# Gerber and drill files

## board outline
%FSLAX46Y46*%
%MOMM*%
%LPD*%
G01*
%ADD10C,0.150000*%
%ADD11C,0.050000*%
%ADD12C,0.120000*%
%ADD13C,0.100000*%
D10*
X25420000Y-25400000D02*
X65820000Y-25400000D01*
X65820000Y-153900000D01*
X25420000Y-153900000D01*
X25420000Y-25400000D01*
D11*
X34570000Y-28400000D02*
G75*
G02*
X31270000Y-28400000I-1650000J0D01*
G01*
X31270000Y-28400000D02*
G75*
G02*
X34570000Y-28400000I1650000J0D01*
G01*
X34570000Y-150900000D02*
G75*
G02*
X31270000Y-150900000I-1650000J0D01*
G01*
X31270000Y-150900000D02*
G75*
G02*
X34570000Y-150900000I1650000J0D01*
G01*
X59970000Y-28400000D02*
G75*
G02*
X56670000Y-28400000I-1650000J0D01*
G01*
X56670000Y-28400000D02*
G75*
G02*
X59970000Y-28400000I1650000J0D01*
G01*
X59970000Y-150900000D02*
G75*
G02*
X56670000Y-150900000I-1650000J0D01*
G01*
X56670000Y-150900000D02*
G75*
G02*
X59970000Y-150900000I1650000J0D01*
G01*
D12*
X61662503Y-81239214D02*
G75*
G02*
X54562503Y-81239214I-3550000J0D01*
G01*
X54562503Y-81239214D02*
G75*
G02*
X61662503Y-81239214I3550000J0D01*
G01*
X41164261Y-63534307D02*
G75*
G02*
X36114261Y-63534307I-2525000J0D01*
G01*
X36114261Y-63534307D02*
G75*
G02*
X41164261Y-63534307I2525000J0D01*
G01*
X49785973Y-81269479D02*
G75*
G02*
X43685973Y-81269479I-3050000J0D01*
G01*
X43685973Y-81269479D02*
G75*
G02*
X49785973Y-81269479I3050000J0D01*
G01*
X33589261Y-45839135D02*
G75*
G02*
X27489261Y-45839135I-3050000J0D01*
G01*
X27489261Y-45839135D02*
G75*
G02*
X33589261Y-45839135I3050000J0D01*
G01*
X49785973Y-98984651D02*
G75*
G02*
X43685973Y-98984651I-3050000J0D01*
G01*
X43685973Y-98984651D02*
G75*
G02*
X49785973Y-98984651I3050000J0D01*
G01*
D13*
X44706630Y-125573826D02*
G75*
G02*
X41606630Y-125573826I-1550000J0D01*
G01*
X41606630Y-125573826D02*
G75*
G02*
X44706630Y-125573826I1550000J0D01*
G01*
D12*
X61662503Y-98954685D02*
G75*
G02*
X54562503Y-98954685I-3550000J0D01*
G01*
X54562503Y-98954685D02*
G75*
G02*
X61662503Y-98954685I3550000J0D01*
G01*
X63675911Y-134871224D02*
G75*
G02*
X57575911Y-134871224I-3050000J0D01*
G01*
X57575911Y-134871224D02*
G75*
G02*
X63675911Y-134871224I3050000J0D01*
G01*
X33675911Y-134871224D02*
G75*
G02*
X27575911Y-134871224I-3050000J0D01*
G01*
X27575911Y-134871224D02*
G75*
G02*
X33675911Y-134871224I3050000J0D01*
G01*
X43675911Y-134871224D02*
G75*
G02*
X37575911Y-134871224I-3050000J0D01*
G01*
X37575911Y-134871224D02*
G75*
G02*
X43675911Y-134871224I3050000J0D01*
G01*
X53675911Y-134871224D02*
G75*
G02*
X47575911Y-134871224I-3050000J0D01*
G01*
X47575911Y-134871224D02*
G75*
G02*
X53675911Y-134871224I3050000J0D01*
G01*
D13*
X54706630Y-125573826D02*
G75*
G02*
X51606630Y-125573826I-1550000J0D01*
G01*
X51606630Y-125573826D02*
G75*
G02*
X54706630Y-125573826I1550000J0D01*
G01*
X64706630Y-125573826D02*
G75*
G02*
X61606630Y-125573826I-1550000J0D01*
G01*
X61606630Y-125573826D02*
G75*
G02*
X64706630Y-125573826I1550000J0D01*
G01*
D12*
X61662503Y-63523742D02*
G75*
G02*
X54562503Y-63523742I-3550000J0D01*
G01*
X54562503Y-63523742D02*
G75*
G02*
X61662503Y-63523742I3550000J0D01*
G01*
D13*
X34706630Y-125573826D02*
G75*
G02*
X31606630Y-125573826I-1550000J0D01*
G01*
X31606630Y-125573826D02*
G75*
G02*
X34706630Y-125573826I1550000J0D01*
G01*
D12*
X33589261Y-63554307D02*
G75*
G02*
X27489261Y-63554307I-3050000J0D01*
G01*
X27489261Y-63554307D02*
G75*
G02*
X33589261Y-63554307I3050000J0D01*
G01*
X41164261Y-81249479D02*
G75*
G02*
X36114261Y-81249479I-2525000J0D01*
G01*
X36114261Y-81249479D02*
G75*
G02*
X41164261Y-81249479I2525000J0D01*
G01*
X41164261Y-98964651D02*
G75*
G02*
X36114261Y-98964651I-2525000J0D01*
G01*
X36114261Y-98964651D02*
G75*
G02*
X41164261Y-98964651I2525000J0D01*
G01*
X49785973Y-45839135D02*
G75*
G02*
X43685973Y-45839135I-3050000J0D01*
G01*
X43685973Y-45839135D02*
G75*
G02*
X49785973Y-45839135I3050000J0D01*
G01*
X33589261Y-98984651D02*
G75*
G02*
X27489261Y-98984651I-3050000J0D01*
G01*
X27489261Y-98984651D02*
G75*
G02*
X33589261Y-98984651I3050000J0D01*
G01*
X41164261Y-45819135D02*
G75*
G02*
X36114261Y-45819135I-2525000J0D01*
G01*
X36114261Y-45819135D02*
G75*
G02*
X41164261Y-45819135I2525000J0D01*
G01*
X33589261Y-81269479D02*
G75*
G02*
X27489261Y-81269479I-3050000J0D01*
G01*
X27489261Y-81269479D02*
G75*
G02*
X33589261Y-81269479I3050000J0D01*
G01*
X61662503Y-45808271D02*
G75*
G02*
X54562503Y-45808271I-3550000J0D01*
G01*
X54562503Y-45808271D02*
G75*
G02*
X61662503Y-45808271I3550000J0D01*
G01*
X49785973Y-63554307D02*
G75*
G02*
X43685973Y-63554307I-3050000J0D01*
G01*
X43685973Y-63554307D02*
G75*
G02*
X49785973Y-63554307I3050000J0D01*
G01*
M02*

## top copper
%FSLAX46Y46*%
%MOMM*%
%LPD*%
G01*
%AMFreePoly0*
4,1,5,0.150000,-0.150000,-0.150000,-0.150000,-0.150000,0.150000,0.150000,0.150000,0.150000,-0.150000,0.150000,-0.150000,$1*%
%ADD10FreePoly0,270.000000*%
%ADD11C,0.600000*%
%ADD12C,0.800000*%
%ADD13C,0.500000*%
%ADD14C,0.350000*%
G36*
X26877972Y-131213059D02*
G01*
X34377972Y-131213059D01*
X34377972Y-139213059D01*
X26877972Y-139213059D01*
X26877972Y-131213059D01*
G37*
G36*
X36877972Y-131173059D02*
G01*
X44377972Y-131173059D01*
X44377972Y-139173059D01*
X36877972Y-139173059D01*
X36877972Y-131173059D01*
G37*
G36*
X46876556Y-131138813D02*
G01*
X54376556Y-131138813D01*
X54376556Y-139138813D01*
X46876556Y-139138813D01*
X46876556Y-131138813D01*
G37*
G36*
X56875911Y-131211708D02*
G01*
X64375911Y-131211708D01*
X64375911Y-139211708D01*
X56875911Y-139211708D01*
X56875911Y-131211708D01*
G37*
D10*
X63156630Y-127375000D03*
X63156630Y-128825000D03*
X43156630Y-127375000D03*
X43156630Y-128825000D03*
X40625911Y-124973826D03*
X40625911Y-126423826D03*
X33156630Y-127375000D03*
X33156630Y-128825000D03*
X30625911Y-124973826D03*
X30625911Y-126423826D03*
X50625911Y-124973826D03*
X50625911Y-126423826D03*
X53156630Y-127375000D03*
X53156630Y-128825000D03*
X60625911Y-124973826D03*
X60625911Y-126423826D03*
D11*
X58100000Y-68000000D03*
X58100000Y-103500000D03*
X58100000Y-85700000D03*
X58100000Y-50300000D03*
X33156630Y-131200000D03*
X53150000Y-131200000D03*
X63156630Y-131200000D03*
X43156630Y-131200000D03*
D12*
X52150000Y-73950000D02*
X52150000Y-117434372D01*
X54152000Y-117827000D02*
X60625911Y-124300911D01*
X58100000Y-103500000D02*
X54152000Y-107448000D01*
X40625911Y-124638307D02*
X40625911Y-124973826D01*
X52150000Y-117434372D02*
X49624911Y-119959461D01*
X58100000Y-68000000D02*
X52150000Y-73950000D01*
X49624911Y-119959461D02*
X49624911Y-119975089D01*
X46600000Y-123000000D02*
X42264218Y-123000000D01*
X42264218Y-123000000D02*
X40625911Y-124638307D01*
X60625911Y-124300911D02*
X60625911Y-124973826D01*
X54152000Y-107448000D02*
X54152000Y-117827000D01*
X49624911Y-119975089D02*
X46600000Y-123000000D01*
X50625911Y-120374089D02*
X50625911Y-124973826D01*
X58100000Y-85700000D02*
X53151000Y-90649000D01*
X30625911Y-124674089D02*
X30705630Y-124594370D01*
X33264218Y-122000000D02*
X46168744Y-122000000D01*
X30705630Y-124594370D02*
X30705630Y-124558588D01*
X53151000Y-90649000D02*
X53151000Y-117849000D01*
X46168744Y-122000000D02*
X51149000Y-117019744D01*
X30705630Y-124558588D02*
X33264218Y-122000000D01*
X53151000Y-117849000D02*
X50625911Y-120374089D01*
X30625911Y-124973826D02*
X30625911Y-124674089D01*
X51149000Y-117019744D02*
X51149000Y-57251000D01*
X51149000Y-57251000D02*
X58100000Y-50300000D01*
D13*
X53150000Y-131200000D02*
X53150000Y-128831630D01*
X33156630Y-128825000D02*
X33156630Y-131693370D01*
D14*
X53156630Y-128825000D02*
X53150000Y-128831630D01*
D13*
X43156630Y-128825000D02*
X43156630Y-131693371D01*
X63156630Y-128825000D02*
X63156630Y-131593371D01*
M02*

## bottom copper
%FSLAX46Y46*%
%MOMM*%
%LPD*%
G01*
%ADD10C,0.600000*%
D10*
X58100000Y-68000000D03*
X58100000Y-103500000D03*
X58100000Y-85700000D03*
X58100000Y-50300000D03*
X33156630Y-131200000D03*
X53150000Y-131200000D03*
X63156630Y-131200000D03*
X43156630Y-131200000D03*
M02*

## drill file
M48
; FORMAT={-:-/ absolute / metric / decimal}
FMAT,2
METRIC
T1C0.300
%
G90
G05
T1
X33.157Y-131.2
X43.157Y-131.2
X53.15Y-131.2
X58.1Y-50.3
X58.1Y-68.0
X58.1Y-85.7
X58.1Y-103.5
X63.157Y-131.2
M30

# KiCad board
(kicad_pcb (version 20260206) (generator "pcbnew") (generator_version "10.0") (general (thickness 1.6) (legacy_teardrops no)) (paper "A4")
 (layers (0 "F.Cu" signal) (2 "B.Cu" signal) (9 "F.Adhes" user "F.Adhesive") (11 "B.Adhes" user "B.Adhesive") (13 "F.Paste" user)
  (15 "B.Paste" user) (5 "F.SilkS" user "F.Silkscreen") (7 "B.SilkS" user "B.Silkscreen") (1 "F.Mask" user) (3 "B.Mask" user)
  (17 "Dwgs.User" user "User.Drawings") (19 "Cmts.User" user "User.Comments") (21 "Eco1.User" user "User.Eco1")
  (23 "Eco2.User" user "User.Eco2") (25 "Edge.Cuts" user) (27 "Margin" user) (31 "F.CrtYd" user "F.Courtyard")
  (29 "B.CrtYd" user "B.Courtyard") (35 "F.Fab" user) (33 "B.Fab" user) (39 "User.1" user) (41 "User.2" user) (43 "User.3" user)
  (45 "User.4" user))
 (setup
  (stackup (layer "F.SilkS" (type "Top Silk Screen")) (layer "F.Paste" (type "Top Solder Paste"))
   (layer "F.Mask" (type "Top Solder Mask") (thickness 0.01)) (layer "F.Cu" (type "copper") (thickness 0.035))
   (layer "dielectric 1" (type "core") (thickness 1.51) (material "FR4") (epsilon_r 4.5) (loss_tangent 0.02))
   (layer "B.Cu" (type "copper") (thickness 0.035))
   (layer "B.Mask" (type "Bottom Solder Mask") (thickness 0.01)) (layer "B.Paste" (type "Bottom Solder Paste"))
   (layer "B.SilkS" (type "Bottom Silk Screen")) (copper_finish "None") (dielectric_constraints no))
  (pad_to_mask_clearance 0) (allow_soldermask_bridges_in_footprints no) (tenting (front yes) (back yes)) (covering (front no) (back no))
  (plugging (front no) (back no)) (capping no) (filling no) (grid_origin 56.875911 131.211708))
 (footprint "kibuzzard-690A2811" (layer "F.Cu") (at 27.621439 39.2)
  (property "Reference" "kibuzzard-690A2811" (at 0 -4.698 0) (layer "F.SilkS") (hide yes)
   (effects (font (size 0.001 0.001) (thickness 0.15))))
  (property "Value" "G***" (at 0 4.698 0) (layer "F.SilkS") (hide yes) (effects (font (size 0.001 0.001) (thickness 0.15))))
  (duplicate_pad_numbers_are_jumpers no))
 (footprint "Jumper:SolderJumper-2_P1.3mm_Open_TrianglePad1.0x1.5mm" (layer "F.Cu") (at 63.15663 128.1 -90)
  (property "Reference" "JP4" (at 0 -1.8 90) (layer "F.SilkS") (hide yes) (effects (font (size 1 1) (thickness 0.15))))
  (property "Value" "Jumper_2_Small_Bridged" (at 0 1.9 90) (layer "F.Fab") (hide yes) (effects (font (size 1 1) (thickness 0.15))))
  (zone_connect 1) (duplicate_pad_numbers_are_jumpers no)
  (pad "1" smd custom (at -0.725 0 270) (size 0.3 0.3) (layers "F.Cu" "F.Mask") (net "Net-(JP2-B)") (zone_connect 2)
   (thermal_bridge_angle 45) (options (clearance outline) (anchor rect)) (primitives))
  (pad "2" smd custom (at 0.725 0 270) (size 0.3 0.3) (layers "F.Cu" "F.Mask") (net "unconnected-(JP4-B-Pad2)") (zone_connect 2)
   (thermal_bridge_angle 45) (options (clearance outline) (anchor rect)) (primitives)))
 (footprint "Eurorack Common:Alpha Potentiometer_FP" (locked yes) (layer "F.Cu") (at 55.612503 88.849214)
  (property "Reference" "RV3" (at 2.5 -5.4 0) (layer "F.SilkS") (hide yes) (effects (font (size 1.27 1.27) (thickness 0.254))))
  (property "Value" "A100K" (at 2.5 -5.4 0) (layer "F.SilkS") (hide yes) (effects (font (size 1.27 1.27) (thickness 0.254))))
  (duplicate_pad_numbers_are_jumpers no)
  (fp_circle (center 2.5 -7.61) (end 6.05 -7.61) (stroke (width 0.12) (type solid)) (fill no) (layer "Edge.Cuts")))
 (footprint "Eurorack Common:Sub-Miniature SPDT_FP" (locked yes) (layer "F.Cu") (at 38.639261 63.534307 90)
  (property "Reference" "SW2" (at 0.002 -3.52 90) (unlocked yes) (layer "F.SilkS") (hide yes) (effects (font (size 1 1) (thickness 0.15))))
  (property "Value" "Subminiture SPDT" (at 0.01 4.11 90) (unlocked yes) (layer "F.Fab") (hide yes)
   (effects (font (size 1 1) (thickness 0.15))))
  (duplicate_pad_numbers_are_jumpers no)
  (fp_circle (center 0 0) (end 2.525 0) (stroke (width 0.12) (type solid)) (fill no) (layer "Edge.Cuts")))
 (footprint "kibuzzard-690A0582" (layer "F.Cu") (at 41.52 141.85)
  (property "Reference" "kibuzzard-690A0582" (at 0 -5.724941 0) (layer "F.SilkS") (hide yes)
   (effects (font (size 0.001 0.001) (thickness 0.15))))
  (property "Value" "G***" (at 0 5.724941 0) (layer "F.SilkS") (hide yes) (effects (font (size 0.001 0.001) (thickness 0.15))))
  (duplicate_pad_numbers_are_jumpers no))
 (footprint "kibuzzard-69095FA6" (layer "F.Cu") (at 30.670922 113.458966)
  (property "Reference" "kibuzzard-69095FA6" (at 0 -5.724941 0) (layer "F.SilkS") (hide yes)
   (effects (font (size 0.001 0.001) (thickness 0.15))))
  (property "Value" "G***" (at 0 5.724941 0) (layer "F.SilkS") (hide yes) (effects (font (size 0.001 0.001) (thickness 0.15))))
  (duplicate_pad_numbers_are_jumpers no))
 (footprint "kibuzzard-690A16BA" (layer "F.Cu") (at 46.3 113.458966)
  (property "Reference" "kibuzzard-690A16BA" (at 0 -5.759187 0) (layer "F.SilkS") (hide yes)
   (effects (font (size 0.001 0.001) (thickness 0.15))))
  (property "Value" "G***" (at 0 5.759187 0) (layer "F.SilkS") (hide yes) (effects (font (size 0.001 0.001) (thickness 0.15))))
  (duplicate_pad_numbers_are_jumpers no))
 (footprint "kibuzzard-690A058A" (layer "F.Cu") (at 51.53 141.85)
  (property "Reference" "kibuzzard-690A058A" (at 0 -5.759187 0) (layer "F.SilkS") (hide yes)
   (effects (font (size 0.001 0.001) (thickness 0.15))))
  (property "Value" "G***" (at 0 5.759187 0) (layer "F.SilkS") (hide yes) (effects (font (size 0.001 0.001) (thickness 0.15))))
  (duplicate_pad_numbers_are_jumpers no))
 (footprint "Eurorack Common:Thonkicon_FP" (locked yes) (layer "F.Cu") (at 46.735973 74.789479)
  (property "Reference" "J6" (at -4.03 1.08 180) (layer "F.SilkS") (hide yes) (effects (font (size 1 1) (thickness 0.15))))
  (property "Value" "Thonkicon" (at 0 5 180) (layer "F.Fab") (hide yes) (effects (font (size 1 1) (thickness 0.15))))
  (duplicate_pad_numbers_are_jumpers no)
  (fp_circle (center 0 6.48) (end 3.05 6.48) (stroke (width 0.12) (type solid)) (fill no) (layer "Edge.Cuts")))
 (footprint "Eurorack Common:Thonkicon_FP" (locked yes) (layer "F.Cu") (at 30.539261 39.359135)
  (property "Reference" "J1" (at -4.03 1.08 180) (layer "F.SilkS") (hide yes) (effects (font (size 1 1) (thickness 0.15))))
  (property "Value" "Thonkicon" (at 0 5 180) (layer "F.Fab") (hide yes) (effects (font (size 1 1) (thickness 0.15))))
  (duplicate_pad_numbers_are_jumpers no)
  (fp_circle (center 0 6.48) (end 3.05 6.48) (stroke (width 0.12) (type solid)) (fill no) (layer "Edge.Cuts")))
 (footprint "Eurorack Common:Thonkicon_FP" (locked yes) (layer "F.Cu") (at 46.735973 92.504651)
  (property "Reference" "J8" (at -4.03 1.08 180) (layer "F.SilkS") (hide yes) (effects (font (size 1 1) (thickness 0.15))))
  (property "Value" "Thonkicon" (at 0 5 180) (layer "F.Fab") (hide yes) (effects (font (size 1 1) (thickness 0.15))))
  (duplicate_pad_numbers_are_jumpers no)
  (fp_circle (center 0 6.48) (end 3.05 6.48) (stroke (width 0.12) (type solid)) (fill no) (layer "Edge.Cuts")))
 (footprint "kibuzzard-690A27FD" (layer "F.Cu") (at 27.429315 56.9)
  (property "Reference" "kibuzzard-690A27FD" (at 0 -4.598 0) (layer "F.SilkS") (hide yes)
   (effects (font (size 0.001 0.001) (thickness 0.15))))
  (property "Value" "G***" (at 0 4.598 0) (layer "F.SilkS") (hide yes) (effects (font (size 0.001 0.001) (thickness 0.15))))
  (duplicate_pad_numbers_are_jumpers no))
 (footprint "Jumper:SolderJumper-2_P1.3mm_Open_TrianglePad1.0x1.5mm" (layer "F.Cu") (at 43.15663 128.1 -90)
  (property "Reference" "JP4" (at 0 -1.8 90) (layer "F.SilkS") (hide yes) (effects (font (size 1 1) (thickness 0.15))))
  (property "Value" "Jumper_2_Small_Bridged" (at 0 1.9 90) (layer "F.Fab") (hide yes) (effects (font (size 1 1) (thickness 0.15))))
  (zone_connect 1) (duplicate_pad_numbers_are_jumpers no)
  (pad "1" smd custom (at -0.725 0 270) (size 0.3 0.3) (layers "F.Cu" "F.Mask") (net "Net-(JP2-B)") (zone_connect 2)
   (thermal_bridge_angle 45) (options (clearance outline) (anchor rect)) (primitives))
  (pad "2" smd custom (at 0.725 0 270) (size 0.3 0.3) (layers "F.Cu" "F.Mask") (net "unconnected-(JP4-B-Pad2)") (zone_connect 2)
   (thermal_bridge_angle 45) (options (clearance outline) (anchor rect)) (primitives)))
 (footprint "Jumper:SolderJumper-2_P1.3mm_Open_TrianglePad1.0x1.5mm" (layer "F.Cu") (at 40.625911 125.698826 -90)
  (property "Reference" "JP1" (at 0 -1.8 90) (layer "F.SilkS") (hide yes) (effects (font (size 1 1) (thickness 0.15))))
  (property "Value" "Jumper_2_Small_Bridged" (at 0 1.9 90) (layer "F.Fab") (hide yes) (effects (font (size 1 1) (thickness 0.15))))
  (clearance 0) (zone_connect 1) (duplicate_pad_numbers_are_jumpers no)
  (pad "1" smd custom (at -0.725 0 270) (size 0.3 0.3) (layers "F.Cu" "F.Mask") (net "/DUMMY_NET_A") (zone_connect 2)
   (thermal_bridge_angle 45) (options (clearance outline) (anchor rect)) (primitives))
  (pad "2" smd custom (at 0.725 0 270) (size 0.3 0.3) (layers "F.Cu" "F.Mask") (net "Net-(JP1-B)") (zone_connect 2)
   (thermal_bridge_angle 45) (options (clearance outline) (anchor rect)) (primitives)))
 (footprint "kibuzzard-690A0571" (layer "F.Cu") (at 31.52 141.89)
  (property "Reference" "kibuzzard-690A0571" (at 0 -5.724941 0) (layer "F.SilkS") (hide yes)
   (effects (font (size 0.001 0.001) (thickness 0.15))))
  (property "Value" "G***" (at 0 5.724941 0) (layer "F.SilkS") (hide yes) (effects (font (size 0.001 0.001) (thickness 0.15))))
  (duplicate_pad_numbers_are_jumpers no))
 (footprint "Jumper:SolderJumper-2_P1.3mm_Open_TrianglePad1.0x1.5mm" (layer "F.Cu") (at 33.15663 128.1 -90)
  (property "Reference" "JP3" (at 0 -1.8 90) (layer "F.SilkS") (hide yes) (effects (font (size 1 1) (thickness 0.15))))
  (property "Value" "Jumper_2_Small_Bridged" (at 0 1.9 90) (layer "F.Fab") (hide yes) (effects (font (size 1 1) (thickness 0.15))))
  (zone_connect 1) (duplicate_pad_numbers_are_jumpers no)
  (pad "1" smd custom (at -0.725 0 270) (size 0.3 0.3) (layers "F.Cu" "F.Mask") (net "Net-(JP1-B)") (zone_connect 2)
   (thermal_bridge_angle 45) (options (clearance outline) (anchor rect)) (primitives))
  (pad "2" smd custom (at 0.725 0 270) (size 0.3 0.3) (layers "F.Cu" "F.Mask") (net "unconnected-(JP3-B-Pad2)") (zone_connect 2)
   (thermal_bridge_angle 45) (options (clearance outline) (anchor rect)) (primitives)))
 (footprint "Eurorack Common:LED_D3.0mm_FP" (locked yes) (layer "F.Cu") (at 43.15663 124.303826 -90)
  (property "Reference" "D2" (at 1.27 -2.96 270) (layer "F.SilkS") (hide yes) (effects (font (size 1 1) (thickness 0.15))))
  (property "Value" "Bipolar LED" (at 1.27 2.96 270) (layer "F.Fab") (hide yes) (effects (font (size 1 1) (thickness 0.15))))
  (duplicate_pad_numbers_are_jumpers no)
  (fp_circle (center 1.27 0) (end 2.82 0) (stroke (width 0.1) (type solid)) (fill no) (layer "Edge.Cuts")))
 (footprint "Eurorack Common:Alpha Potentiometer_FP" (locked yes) (layer "F.Cu") (at 55.612503 106.564685)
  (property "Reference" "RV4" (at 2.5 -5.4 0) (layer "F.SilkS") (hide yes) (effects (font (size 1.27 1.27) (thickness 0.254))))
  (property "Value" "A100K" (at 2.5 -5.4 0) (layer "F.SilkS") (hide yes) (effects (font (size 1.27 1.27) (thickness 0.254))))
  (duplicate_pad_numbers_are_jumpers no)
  (fp_circle (center 2.5 -7.61) (end 6.05 -7.61) (stroke (width 0.12) (type solid)) (fill no) (layer "Edge.Cuts")))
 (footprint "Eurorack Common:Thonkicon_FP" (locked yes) (layer "F.Cu") (at 60.625911 128.391224)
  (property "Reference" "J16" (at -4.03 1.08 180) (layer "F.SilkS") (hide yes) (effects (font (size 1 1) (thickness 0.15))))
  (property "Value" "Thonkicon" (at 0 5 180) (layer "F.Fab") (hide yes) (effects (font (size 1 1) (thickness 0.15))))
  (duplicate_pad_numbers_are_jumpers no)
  (fp_circle (center 0 6.48) (end 3.05 6.48) (stroke (width 0.12) (type solid)) (fill no) (layer "Edge.Cuts")))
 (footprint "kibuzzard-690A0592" (layer "F.Cu") (at 60.625911 141.888649)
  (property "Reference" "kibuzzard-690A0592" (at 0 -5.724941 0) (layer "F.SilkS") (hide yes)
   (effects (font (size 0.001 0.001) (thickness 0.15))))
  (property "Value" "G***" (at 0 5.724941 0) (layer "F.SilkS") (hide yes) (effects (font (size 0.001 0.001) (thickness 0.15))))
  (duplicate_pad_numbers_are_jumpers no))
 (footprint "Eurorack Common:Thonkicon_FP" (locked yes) (layer "F.Cu") (at 30.625911 128.391224)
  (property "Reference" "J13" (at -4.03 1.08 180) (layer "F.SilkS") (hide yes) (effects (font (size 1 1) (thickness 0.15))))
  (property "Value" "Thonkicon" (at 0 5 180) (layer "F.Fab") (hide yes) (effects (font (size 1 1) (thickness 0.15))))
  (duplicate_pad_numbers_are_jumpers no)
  (fp_circle (center 0 6.48) (end 3.05 6.48) (stroke (width 0.12) (type solid)) (fill no) (layer "Edge.Cuts")))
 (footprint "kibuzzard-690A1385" (layer "F.Cu") (at 59.8 113.458966)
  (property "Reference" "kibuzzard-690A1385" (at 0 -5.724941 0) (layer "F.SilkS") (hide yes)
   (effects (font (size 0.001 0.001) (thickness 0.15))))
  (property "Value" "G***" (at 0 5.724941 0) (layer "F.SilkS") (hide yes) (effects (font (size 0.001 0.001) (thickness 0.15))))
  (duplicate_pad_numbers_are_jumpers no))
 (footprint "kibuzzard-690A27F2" (layer "F.Cu") (at 27.481302 74.6)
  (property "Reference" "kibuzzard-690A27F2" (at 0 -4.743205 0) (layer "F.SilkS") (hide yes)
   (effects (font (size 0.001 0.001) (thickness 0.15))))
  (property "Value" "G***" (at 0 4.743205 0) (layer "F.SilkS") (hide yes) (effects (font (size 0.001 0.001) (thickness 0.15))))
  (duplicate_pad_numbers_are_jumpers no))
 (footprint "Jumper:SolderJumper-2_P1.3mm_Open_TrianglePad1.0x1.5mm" (layer "F.Cu") (at 30.625911 125.698826 -90)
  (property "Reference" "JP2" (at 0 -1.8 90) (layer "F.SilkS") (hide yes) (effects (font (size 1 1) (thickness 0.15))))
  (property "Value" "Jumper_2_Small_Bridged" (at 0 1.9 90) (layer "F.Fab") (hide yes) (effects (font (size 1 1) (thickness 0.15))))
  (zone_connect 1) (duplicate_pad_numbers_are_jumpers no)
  (pad "1" smd custom (at -0.725 0 270) (size 0.3 0.3) (layers "F.Cu" "F.Mask") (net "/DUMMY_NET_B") (zone_connect 2)
   (thermal_bridge_angle 45) (options (clearance outline) (anchor rect)) (primitives))
  (pad "2" smd custom (at 0.725 0 270) (size 0.3 0.3) (layers "F.Cu" "F.Mask") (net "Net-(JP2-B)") (zone_connect 2)
   (thermal_bridge_angle 45) (options (clearance outline) (anchor rect)) (primitives)))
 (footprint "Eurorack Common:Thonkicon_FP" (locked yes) (layer "F.Cu") (at 40.625911 128.391224)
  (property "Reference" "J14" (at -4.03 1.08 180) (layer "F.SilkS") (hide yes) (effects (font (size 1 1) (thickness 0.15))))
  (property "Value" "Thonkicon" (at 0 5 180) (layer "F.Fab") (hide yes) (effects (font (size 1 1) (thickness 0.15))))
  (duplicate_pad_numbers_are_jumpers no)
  (fp_circle (center 0 6.48) (end 3.05 6.48) (stroke (width 0.12) (type solid)) (fill no) (layer "Edge.Cuts")))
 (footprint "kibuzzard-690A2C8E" (layer "F.Cu") (at 45.67177 34.65)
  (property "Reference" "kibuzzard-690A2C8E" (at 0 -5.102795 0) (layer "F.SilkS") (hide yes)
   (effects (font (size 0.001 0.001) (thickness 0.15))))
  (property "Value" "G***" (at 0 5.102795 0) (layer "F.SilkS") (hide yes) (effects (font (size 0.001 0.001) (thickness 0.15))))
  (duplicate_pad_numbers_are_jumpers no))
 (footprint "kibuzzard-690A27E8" (layer "F.Cu") (at 27.483562 92.2)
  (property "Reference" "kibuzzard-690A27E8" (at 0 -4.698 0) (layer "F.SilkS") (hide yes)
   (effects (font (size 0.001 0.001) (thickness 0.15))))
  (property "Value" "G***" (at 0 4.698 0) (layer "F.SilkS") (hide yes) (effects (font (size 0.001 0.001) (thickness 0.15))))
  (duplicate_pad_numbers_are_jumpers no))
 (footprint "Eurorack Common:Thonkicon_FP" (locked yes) (layer "F.Cu") (at 50.625911 128.391224)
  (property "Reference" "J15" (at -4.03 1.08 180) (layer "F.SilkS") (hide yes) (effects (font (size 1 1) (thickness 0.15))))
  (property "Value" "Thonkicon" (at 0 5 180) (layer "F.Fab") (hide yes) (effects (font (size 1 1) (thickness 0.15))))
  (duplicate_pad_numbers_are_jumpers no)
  (fp_circle (center 0 6.48) (end 3.05 6.48) (stroke (width 0.12) (type solid)) (fill no) (layer "Edge.Cuts")))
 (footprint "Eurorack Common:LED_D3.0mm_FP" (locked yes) (layer "F.Cu") (at 53.15663 124.303826 -90)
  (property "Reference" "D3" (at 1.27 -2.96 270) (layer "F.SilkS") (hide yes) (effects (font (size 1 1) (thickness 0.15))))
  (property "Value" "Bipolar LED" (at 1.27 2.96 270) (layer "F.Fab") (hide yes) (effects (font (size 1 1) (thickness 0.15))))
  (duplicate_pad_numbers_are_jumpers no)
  (fp_circle (center 1.27 0) (end 2.82 0) (stroke (width 0.1) (type solid)) (fill no) (layer "Edge.Cuts")))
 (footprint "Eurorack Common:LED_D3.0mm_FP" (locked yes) (layer "F.Cu") (at 63.15663 124.303826 -90)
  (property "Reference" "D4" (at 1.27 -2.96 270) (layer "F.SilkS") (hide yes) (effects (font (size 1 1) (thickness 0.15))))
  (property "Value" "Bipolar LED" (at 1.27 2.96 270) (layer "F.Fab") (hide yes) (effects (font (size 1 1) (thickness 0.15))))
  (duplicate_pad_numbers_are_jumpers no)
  (fp_circle (center 1.27 0) (end 2.82 0) (stroke (width 0.1) (type solid)) (fill no) (layer "Edge.Cuts")))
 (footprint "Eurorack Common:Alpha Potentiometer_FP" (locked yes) (layer "F.Cu") (at 55.612503 71.133742)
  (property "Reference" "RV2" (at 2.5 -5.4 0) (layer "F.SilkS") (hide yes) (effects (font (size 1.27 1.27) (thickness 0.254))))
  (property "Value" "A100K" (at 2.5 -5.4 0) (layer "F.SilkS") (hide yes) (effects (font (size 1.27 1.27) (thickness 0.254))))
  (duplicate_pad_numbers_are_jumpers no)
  (fp_circle (center 2.5 -7.61) (end 6.05 -7.61) (stroke (width 0.12) (type solid)) (fill no) (layer "Edge.Cuts")))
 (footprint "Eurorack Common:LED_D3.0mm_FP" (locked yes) (layer "F.Cu") (at 33.15663 124.303826 -90)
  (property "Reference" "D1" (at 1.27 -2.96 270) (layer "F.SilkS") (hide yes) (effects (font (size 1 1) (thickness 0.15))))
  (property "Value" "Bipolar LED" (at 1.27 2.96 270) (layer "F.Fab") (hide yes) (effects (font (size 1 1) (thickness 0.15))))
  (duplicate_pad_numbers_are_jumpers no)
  (fp_circle (center 1.27 0) (end 2.82 0) (stroke (width 0.1) (type solid)) (fill no) (layer "Edge.Cuts")))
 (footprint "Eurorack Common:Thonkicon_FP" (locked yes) (layer "F.Cu") (at 30.539261 57.074307)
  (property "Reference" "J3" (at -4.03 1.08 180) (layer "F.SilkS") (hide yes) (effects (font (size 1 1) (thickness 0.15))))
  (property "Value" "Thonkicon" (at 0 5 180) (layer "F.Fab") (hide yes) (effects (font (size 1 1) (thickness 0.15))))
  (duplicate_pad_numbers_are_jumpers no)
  (fp_circle (center 0 6.48) (end 3.05 6.48) (stroke (width 0.12) (type solid)) (fill no) (layer "Edge.Cuts")))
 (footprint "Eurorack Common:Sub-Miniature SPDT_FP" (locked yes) (layer "F.Cu") (at 38.639261 81.249479 90)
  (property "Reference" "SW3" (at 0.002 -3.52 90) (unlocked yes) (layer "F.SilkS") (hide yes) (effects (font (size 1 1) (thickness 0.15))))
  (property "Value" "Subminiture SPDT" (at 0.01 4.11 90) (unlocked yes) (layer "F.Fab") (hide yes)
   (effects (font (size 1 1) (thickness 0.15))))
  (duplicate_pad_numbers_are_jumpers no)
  (fp_circle (center 0 0) (end 2.525 0) (stroke (width 0.12) (type solid)) (fill no) (layer "Edge.Cuts")))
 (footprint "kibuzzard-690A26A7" (layer "F.Cu") (at 38.520101 113.458966)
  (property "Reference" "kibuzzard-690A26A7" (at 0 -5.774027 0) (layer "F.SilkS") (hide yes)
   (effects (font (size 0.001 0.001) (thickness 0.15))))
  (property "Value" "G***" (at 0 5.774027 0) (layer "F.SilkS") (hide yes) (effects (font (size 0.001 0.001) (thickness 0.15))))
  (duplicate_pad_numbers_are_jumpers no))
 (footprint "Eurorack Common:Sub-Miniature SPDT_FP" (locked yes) (layer "F.Cu") (at 38.639261 98.964651 90)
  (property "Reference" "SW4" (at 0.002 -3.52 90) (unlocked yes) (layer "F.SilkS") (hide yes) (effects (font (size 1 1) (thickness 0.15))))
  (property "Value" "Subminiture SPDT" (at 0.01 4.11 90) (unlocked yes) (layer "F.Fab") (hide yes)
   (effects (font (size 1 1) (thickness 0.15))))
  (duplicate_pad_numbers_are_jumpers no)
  (fp_circle (center 0 0) (end 2.525 0) (stroke (width 0.12) (type solid)) (fill no) (layer "Edge.Cuts")))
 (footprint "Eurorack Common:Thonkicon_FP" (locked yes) (layer "F.Cu") (at 46.735973 39.359135)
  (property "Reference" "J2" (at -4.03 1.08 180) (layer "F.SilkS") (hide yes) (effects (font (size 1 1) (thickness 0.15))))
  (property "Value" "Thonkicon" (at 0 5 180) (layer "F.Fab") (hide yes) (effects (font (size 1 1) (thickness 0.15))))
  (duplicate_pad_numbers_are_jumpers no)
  (fp_circle (center 0 6.48) (end 3.05 6.48) (stroke (width 0.12) (type solid)) (fill no) (layer "Edge.Cuts")))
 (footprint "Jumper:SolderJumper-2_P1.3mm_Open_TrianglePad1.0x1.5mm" (layer "F.Cu") (at 50.625911 125.698826 -90)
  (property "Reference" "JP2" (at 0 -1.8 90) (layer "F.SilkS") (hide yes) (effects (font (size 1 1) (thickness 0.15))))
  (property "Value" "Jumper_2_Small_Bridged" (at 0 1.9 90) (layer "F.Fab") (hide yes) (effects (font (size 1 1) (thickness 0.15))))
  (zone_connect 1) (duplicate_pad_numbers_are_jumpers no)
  (pad "1" smd custom (at -0.725 0 270) (size 0.3 0.3) (layers "F.Cu" "F.Mask") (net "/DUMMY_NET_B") (zone_connect 2)
   (thermal_bridge_angle 45) (options (clearance outline) (anchor rect)) (primitives))
  (pad "2" smd custom (at 0.725 0 270) (size 0.3 0.3) (layers "F.Cu" "F.Mask") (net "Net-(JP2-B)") (zone_connect 2)
   (thermal_bridge_angle 45) (options (clearance outline) (anchor rect)) (primitives)))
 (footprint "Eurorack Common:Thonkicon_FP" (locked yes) (layer "F.Cu") (at 30.539261 92.504651)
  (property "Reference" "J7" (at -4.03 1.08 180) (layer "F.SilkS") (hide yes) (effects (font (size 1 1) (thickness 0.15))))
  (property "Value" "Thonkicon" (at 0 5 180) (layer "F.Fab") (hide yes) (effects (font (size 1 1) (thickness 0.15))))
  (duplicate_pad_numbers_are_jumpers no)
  (fp_circle (center 0 6.48) (end 3.05 6.48) (stroke (width 0.12) (type solid)) (fill no) (layer "Edge.Cuts")))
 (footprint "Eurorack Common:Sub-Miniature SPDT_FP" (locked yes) (layer "F.Cu") (at 38.639261 45.819135 90)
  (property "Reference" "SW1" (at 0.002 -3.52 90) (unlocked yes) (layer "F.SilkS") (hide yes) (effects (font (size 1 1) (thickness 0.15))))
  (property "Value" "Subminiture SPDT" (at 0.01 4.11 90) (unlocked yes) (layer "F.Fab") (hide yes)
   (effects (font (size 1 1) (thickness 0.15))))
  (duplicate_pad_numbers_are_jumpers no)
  (fp_circle (center 0 0) (end 2.525 0) (stroke (width 0.12) (type solid)) (fill no) (layer "Edge.Cuts")))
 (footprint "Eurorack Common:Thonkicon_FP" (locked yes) (layer "F.Cu") (at 30.539261 74.789479)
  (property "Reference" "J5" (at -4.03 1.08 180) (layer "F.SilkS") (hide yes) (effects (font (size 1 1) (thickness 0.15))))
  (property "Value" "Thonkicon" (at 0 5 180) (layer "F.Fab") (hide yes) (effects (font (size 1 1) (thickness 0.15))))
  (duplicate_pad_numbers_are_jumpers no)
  (fp_circle (center 0 6.48) (end 3.05 6.48) (stroke (width 0.12) (type solid)) (fill no) (layer "Edge.Cuts")))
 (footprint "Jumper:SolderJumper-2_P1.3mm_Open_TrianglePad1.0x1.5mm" (layer "F.Cu") (at 53.15663 128.1 -90)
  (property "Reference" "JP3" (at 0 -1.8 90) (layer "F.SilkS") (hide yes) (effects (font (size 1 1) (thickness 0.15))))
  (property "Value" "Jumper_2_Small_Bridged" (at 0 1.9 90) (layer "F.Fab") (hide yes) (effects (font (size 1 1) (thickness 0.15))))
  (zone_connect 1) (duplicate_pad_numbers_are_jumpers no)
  (pad "1" smd custom (at -0.725 0 270) (size 0.3 0.3) (layers "F.Cu" "F.Mask") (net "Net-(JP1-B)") (zone_connect 2)
   (thermal_bridge_angle 45) (options (clearance outline) (anchor rect)) (primitives))
  (pad "2" smd custom (at 0.725 0 270) (size 0.3 0.3) (layers "F.Cu" "F.Mask") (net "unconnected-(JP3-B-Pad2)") (zone_connect 2)
   (thermal_bridge_angle 45) (options (clearance outline) (anchor rect)) (primitives)))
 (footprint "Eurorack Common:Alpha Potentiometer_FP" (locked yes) (layer "F.Cu") (at 55.612503 53.418271)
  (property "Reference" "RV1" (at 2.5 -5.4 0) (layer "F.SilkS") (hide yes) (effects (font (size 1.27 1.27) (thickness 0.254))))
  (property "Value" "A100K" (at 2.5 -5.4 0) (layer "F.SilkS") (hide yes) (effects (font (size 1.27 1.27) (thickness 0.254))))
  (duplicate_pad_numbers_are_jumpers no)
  (fp_circle (center 2.5 -7.61) (end 6.05 -7.61) (stroke (width 0.12) (type solid)) (fill no) (layer "Edge.Cuts")))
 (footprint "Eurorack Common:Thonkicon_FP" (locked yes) (layer "F.Cu") (at 46.735973 57.074307)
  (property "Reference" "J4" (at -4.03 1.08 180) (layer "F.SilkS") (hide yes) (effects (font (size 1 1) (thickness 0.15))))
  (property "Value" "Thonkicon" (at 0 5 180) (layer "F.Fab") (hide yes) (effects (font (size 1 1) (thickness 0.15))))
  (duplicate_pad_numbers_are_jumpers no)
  (fp_circle (center 0 6.48) (end 3.05 6.48) (stroke (width 0.12) (type solid)) (fill no) (layer "Edge.Cuts")))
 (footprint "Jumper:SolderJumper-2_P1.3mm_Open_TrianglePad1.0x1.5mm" (layer "F.Cu") (at 60.625911 125.698826 -90)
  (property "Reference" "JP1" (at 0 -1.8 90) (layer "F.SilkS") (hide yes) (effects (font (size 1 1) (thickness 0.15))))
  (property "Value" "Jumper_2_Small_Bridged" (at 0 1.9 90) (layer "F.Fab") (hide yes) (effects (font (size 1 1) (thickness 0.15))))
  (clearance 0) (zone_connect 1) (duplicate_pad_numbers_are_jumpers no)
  (pad "1" smd custom (at -0.725 0 270) (size 0.3 0.3) (layers "F.Cu" "F.Mask") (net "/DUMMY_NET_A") (zone_connect 2)
   (thermal_bridge_angle 45) (options (clearance outline) (anchor rect)) (primitives))
  (pad "2" smd custom (at 0.725 0 270) (size 0.3 0.3) (layers "F.Cu" "F.Mask") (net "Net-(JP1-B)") (zone_connect 2)
   (thermal_bridge_angle 45) (options (clearance outline) (anchor rect)) (primitives)))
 (gr_rect (start 26.877972 131.213059) (end 34.377972 139.213059) (stroke (width 0) (type solid)) (fill yes) (layers "F.Cu" "F.Mask")
  (net "unconnected-(JP3-B-Pad2)"))
 (gr_rect (start 36.877972 131.173059) (end 44.377972 139.173059) (stroke (width 0) (type solid)) (fill yes) (layers "F.Cu" "F.Mask")
  (net "unconnected-(JP4-B-Pad2)"))
 (gr_rect (start 46.876556 131.138813) (end 54.376556 139.138813) (stroke (width 0) (type solid)) (fill yes) (layers "F.Cu" "F.Mask")
  (net "unconnected-(JP3-B-Pad2)"))
 (gr_rect (start 56.875911 131.211708) (end 64.375911 139.211708) (stroke (width 0) (type solid)) (fill yes) (layers "F.Cu" "F.Mask")
  (net "unconnected-(JP4-B-Pad2)"))
 (gr_rect (start 25.42 25.4) (end 65.82 153.9) (stroke (width 0.15) (type solid)) (fill no) (layer "Edge.Cuts"))
 (gr_circle (center 32.92 28.4) (end 34.57 28.4) (stroke (width 0.05) (type default)) (fill no) (layer "Edge.Cuts"))
 (gr_circle (center 32.92 150.9) (end 34.57 150.9) (stroke (width 0.05) (type default)) (fill no) (layer "Edge.Cuts"))
 (gr_circle (center 58.32 28.4) (end 59.97 28.4) (stroke (width 0.05) (type default)) (fill no) (layer "Edge.Cuts"))
 (gr_circle (center 58.32 150.9) (end 59.97 150.9) (stroke (width 0.05) (type default)) (fill no) (layer "Edge.Cuts"))
 (segment (start 52.15 73.95) (end 52.15 117.434372) (width 0.8) (layers "F.Cu" "F.Mask") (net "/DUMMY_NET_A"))
 (segment (start 54.152 117.827) (end 60.625911 124.300911) (width 0.8) (layers "F.Cu" "F.Mask") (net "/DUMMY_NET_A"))
 (segment (start 58.1 103.5) (end 54.152 107.448) (width 0.8) (layers "F.Cu" "F.Mask") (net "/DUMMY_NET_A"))
 (segment (start 40.625911 124.638307) (end 40.625911 124.973826) (width 0.8) (layers "F.Cu" "F.Mask") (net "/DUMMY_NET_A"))
 (segment (start 52.15 117.434372) (end 49.624911 119.959461) (width 0.8) (layers "F.Cu" "F.Mask") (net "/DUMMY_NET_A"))
 (segment (start 58.1 68) (end 52.15 73.95) (width 0.8) (layers "F.Cu" "F.Mask") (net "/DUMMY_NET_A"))
 (segment (start 49.624911 119.959461) (end 49.624911 119.975089) (width 0.8) (layers "F.Cu" "F.Mask") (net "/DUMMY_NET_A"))
 (segment (start 46.6 123) (end 42.264218 123) (width 0.8) (layers "F.Cu" "F.Mask") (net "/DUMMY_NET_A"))
 (segment (start 42.264218 123) (end 40.625911 124.638307) (width 0.8) (layers "F.Cu" "F.Mask") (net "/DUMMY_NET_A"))
 (segment (start 60.625911 124.300911) (end 60.625911 124.973826) (width 0.8) (layers "F.Cu" "F.Mask") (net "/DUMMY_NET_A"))
 (segment (start 54.152 107.448) (end 54.152 117.827) (width 0.8) (layers "F.Cu" "F.Mask") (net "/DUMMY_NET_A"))
 (segment (start 49.624911 119.975089) (end 46.6 123) (width 0.8) (layers "F.Cu" "F.Mask") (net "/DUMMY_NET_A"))
 (via (at 58.1 68) (size 0.6) (drill 0.3) (layers "F.Cu" "B.Cu") (free yes) (capping no) (covering (front no) (back no))
  (plugging (front no) (back no)) (filling no) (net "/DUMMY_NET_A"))
 (via (at 58.1 103.5) (size 0.6) (drill 0.3) (layers "F.Cu" "B.Cu") (capping no) (covering (front no) (back no))
  (plugging (front no) (back no)) (filling no) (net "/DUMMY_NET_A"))
 (segment (start 50.625911 120.374089) (end 50.625911 124.973826) (width 0.8) (layers "F.Cu" "F.Mask") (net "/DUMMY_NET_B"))
 (segment (start 58.1 85.7) (end 53.151 90.649) (width 0.8) (layers "F.Cu" "F.Mask") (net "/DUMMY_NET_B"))
 (segment (start 30.625911 124.674089) (end 30.70563 124.59437) (width 0.8) (layer "F.Cu") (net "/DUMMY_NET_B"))
 (segment (start 33.264218 122) (end 46.168744 122) (width 0.8) (layers "F.Cu" "F.Mask") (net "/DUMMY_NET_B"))
 (segment (start 30.70563 124.59437) (end 30.70563 124.558588) (width 0.8) (layer "F.Cu") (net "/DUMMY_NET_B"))
 (segment (start 53.151 90.649) (end 53.151 117.849) (width 0.8) (layers "F.Cu" "F.Mask") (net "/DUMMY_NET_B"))
 (segment (start 46.168744 122) (end 51.149 117.019744) (width 0.8) (layers "F.Cu" "F.Mask") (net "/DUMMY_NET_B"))
 (segment (start 30.70563 124.558588) (end 33.264218 122) (width 0.8) (layers "F.Cu" "F.Mask") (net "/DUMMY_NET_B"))
 (segment (start 53.151 117.849) (end 50.625911 120.374089) (width 0.8) (layers "F.Cu" "F.Mask") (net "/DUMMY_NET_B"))
 (segment (start 30.625911 124.973826) (end 30.625911 124.674089) (width 0.8) (layers "F.Cu" "F.Mask") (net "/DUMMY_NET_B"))
 (segment (start 51.149 117.019744) (end 51.149 57.251) (width 0.8) (layers "F.Cu" "F.Mask") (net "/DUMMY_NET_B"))
 (segment (start 51.149 57.251) (end 58.1 50.3) (width 0.8) (layers "F.Cu" "F.Mask") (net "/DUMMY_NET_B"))
 (via (at 58.1 85.7) (size 0.6) (drill 0.3) (layers "F.Cu" "B.Cu") (free yes) (capping no) (covering (front no) (back no))
  (plugging (front no) (back no)) (filling no) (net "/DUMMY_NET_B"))
 (via (at 58.1 50.3) (size 0.6) (drill 0.3) (layers "F.Cu" "B.Cu") (capping no) (covering (front no) (back no))
  (plugging (front no) (back no)) (filling no) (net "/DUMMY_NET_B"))
 (segment (start 53.15 131.2) (end 53.15 128.83163) (width 0.5) (layers "F.Cu" "F.Mask") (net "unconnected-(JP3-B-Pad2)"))
 (segment (start 33.15663 128.825) (end 33.15663 131.69337) (width 0.5) (layers "F.Cu" "F.Mask") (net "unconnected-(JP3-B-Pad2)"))
 (segment (start 53.15663 128.825) (end 53.15 128.83163) (width 0.35) (layer "F.Cu") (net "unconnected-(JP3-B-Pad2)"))
 (via (at 33.15663 131.2) (size 0.6) (drill 0.3) (layers "F.Cu" "B.Cu") (capping no) (covering (front no) (back no))
  (plugging (front no) (back no)) (filling no) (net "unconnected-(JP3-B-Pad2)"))
 (via (at 53.15 131.2) (size 0.6) (drill 0.3) (layers "F.Cu" "B.Cu") (capping no) (covering (front no) (back no))
  (plugging (front no) (back no)) (filling no) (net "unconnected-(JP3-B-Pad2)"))
 (segment (start 43.15663 128.825) (end 43.15663 131.693371) (width 0.5) (layers "F.Cu" "F.Mask") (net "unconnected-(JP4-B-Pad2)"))
 (segment (start 63.15663 128.825) (end 63.15663 131.593371) (width 0.5) (layers "F.Cu" "F.Mask") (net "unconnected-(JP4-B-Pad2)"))
 (via (at 63.15663 131.2) (size 0.6) (drill 0.3) (layers "F.Cu" "B.Cu") (capping no) (covering (front no) (back no))
  (plugging (front no) (back no)) (filling no) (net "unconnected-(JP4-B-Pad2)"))
 (via (at 43.15663 131.2) (size 0.6) (drill 0.3) (layers "F.Cu" "B.Cu") (capping no) (covering (front no) (back no))
  (plugging (front no) (back no)) (filling no) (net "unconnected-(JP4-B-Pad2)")))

